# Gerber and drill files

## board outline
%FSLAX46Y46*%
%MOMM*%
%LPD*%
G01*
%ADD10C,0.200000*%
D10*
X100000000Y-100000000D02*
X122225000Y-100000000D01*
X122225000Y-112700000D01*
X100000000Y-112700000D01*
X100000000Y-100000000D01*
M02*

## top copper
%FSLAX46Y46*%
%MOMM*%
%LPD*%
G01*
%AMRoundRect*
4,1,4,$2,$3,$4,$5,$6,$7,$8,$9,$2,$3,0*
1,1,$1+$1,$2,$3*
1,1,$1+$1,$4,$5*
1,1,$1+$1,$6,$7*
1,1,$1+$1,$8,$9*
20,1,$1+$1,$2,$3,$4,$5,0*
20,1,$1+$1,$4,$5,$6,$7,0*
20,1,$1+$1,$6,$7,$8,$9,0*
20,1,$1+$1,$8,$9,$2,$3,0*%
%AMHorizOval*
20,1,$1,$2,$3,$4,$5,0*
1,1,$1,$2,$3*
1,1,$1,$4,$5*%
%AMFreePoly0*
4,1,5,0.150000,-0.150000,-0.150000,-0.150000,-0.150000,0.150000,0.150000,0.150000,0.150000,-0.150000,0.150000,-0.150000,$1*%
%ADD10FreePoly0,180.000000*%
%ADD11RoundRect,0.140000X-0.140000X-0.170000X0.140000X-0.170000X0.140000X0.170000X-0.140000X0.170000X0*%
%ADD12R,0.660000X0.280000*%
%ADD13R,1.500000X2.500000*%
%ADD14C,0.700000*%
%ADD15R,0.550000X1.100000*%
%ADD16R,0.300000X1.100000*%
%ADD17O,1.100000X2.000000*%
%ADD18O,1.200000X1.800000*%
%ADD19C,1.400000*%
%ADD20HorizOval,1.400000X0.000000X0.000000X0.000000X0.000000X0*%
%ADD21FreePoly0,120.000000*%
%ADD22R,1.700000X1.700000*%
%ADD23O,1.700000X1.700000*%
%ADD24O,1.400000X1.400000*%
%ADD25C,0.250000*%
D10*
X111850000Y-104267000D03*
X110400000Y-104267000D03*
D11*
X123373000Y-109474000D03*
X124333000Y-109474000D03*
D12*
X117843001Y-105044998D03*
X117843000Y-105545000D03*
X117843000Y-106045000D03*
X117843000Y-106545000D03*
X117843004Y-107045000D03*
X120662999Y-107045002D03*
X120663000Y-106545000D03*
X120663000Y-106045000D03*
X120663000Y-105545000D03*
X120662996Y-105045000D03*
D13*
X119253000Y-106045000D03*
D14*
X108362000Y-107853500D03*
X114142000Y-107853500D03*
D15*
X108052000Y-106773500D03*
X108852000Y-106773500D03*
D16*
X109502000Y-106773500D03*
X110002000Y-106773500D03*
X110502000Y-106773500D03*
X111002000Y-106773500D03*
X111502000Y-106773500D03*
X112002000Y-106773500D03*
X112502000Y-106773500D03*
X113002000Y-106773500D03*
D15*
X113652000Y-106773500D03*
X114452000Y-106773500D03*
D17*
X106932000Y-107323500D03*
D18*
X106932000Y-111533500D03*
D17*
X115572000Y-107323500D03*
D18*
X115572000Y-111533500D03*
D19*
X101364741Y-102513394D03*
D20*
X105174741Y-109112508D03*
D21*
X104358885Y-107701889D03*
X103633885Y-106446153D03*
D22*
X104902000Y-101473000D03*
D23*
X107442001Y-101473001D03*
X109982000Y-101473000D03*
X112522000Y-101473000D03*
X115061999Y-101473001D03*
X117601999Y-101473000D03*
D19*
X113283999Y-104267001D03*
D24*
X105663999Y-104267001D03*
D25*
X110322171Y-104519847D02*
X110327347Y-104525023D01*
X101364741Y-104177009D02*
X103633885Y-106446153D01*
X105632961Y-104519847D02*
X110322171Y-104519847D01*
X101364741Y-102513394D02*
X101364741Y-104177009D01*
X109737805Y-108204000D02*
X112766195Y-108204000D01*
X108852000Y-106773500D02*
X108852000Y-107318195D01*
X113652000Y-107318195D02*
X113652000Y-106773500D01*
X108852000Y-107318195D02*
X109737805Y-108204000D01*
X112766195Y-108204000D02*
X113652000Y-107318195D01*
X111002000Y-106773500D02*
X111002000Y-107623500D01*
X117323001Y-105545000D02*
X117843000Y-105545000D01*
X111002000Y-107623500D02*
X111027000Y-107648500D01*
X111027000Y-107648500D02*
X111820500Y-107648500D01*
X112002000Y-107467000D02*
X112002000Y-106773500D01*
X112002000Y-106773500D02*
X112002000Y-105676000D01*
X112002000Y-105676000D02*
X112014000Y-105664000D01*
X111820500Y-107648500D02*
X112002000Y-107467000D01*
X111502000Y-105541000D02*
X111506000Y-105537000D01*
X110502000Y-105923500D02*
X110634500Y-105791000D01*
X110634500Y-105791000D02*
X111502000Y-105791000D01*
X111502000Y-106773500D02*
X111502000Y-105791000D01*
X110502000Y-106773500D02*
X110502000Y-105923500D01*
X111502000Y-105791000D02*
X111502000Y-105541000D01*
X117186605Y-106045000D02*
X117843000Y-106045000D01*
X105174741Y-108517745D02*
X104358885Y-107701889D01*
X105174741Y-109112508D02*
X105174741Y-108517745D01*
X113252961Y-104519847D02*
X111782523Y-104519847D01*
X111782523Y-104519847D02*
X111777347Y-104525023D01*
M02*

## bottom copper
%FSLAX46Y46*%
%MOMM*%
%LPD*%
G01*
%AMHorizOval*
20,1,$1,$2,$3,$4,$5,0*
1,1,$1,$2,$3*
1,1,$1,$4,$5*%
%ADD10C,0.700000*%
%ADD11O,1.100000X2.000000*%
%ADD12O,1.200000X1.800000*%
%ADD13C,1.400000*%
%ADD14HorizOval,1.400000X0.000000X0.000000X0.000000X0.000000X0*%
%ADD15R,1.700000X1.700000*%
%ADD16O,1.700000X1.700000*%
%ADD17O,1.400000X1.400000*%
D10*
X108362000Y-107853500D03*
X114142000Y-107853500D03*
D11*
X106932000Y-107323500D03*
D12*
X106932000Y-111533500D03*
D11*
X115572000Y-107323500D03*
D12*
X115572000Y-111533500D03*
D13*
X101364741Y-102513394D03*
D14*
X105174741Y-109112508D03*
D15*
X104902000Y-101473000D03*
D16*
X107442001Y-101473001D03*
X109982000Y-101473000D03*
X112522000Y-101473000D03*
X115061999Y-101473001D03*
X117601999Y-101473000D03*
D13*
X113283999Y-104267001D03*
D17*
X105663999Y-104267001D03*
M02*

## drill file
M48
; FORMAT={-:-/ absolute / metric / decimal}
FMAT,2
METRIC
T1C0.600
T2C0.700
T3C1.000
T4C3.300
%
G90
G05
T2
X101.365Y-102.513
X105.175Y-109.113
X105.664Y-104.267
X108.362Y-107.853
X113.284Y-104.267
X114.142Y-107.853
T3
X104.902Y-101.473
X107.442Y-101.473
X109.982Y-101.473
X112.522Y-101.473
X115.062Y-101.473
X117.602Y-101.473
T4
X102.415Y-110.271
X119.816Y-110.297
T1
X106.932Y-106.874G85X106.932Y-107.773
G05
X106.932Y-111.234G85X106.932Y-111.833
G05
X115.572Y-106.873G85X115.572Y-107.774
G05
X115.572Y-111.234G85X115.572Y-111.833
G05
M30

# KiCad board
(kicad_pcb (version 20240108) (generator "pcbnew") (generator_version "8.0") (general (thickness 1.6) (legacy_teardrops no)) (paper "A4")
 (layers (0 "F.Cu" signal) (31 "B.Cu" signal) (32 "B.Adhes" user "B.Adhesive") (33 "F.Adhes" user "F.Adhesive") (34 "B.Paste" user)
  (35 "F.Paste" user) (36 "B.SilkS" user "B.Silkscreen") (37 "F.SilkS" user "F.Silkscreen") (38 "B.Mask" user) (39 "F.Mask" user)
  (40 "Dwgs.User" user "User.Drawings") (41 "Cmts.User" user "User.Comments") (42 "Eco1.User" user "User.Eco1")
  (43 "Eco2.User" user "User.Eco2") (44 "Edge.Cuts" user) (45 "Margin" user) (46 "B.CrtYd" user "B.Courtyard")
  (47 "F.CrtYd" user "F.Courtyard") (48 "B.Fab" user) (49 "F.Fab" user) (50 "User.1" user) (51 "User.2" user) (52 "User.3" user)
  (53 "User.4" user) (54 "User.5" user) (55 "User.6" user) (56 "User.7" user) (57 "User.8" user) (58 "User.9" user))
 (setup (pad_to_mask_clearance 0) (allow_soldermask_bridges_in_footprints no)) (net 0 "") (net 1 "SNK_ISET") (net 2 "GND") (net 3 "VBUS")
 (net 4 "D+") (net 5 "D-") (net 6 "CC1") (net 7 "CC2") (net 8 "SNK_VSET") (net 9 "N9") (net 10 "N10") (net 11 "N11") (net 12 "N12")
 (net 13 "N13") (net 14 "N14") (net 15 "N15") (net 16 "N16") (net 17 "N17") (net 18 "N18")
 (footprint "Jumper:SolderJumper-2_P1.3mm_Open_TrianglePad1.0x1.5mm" (layer "F.Cu") (at 111.125 104.267 180)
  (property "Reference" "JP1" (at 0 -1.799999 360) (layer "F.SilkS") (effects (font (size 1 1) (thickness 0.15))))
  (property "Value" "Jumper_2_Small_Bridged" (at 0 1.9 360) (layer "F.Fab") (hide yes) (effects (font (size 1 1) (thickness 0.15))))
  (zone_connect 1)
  (pad "1" smd custom (at -0.725 0 180) (size 0.3 0.3) (layers "F.Cu" "F.Mask") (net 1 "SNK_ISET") (zone_connect 2)
   (thermal_bridge_angle 45) (options (clearance outline) (anchor rect)) (primitives))
  (pad "2" smd custom (at 0.725 0 180) (size 0.3 0.3) (layers "F.Cu" "F.Mask") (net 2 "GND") (zone_connect 2) (thermal_bridge_angle 45)
   (options (clearance outline) (anchor rect)) (primitives)))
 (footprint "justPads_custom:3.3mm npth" (layer "F.Cu") (at 102.415229 110.27145)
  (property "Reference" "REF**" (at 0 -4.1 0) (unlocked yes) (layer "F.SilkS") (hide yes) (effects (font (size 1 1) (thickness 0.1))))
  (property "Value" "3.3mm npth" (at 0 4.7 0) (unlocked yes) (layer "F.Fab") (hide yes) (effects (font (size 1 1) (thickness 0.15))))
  (pad "" np_thru_hole circle (at 0 0) (size 3.3 3.3) (drill 3.3) (layers "F&B.Cu" "*.Mask")))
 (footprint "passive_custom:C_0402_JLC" (layer "F.Cu") (at 123.8356 109.478)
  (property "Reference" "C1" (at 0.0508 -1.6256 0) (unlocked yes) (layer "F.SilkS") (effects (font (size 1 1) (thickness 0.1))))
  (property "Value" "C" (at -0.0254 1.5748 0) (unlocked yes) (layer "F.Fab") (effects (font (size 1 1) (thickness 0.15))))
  (pad "1" smd roundrect (at -0.4626 -0.004) (size 0.56 0.62) (layers "F.Cu" "F.Paste" "F.Mask") (roundrect_rratio 0.25) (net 2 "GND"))
  (pad "2" smd roundrect (at 0.4974 -0.004) (size 0.56 0.62) (layers "F.Cu" "F.Paste" "F.Mask") (roundrect_rratio 0.25) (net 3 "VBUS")))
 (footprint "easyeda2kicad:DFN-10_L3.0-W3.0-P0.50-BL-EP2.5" (layer "F.Cu") (at 119.253 106.045 -90)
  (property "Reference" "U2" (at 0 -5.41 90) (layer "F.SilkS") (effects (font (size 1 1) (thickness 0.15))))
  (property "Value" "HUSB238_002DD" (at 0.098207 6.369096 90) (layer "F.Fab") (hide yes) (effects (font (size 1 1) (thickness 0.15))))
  (pad "1" smd rect (at -1.000002 1.409999 270) (size 0.28 0.66) (layers "F.Cu" "F.Paste" "F.Mask") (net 3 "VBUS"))
  (pad "2" smd rect (at -0.5 1.41 270) (size 0.28 0.66) (layers "F.Cu" "F.Paste" "F.Mask") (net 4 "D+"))
  (pad "3" smd rect (at 0 1.41 270) (size 0.28 0.66) (layers "F.Cu" "F.Paste" "F.Mask") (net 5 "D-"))
  (pad "4" smd rect (at 0.5 1.41 270) (size 0.28 0.66) (layers "F.Cu" "F.Paste" "F.Mask") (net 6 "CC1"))
  (pad "5" smd rect (at 1 1.409996 270) (size 0.28 0.66) (layers "F.Cu" "F.Paste" "F.Mask") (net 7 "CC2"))
  (pad "6" smd rect (at 1.000002 -1.409999 270) (size 0.28 0.66) (layers "F.Cu" "F.Paste" "F.Mask") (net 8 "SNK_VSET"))
  (pad "7" smd rect (at 0.5 -1.41 270) (size 0.28 0.66) (layers "F.Cu" "F.Paste" "F.Mask") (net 1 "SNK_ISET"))
  (pad "8" smd rect (at 0 -1.41 270) (size 0.28 0.66) (layers "F.Cu" "F.Paste" "F.Mask") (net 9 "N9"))
  (pad "9" smd rect (at -0.5 -1.41 270) (size 0.28 0.66) (layers "F.Cu" "F.Paste" "F.Mask") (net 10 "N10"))
  (pad "10" smd rect (at -1 -1.409996 270) (size 0.28 0.66) (layers "F.Cu" "F.Paste" "F.Mask") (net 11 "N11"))
  (pad "11" smd rect (at 0 0 270) (size 2.5 1.5) (layers "F.Cu" "F.Paste" "F.Mask") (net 2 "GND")))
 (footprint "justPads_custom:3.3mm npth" (layer "F.Cu") (at 119.816242 110.29744)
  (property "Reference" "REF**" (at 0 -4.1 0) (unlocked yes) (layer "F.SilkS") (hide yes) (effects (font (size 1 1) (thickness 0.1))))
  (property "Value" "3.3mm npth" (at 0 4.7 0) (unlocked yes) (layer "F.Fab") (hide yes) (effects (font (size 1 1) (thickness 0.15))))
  (pad "" np_thru_hole circle (at 0 0) (size 3.3 3.3) (drill 3.3) (layers "F&B.Cu" "*.Mask")))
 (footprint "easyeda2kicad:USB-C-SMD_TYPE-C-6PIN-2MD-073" (layer "F.Cu") (at 111.252 109.1535)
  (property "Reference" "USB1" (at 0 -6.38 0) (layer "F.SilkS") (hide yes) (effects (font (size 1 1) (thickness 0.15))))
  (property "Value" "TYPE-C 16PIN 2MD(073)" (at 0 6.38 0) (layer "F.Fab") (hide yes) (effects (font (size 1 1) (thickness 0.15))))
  (pad "" thru_hole circle (at -2.89 -1.3) (size 0.7 0.7) (drill 0.7) (layers "*.Cu" "*.Mask") (remove_unused_layers no))
  (pad "" thru_hole circle (at 2.89 -1.3) (size 0.7 0.7) (drill 0.7) (layers "*.Cu" "*.Mask") (remove_unused_layers no))
  (pad "1" smd rect (at -3.2 -2.38) (size 0.55 1.1) (layers "F.Cu" "F.Paste" "F.Mask") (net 2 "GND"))
  (pad "2" smd rect (at -2.4 -2.38) (size 0.55 1.1) (layers "F.Cu" "F.Paste" "F.Mask") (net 3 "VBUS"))
  (pad "3" smd rect (at -1.75 -2.38) (size 0.3 1.1) (layers "F.Cu" "F.Paste" "F.Mask") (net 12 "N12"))
  (pad "4" smd rect (at -1.25 -2.38) (size 0.3 1.1) (layers "F.Cu" "F.Paste" "F.Mask") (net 6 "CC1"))
  (pad "5" smd rect (at -0.75 -2.38) (size 0.3 1.1) (layers "F.Cu" "F.Paste" "F.Mask") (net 5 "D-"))
  (pad "6" smd rect (at -0.25 -2.38) (size 0.3 1.1) (layers "F.Cu" "F.Paste" "F.Mask") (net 4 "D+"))
  (pad "7" smd rect (at 0.25 -2.38) (size 0.3 1.1) (layers "F.Cu" "F.Paste" "F.Mask") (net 5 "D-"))
  (pad "8" smd rect (at 0.75 -2.38) (size 0.3 1.1) (layers "F.Cu" "F.Paste" "F.Mask") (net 4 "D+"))
  (pad "9" smd rect (at 1.25 -2.38) (size 0.3 1.1) (layers "F.Cu" "F.Paste" "F.Mask") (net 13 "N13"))
  (pad "10" smd rect (at 1.75 -2.38) (size 0.3 1.1) (layers "F.Cu" "F.Paste" "F.Mask") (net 7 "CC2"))
  (pad "11" smd rect (at 2.4 -2.38) (size 0.55 1.1) (layers "F.Cu" "F.Paste" "F.Mask") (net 3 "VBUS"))
  (pad "12" smd rect (at 3.2 -2.38) (size 0.55 1.1) (layers "F.Cu" "F.Paste" "F.Mask") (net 2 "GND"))
  (pad "13" thru_hole oval (at -4.32 -1.83) (size 1.1 2) (drill oval 0.599999 1.499997) (layers "*.Cu" "*.Mask") (remove_unused_layers no)
   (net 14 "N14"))
  (pad "13" thru_hole oval (at -4.32 2.38) (size 1.2 1.8) (drill oval 0.599999 1.199998) (layers "*.Cu" "*.Mask") (remove_unused_layers no)
   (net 14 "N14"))
  (pad "14" thru_hole oval (at 4.32 -1.83) (size 1.1 2) (drill oval 0.599999 1.500022) (layers "*.Cu" "*.Mask") (remove_unused_layers no)
   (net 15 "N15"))
  (pad "14" thru_hole oval (at 4.32 2.38) (size 1.2 1.8) (drill oval 0.599999 1.199998) (layers "*.Cu" "*.Mask") (remove_unused_layers no)
   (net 15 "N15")))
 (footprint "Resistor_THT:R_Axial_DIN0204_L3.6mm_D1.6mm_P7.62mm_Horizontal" (layer "F.Cu") (at 101.364741 102.513394 -60)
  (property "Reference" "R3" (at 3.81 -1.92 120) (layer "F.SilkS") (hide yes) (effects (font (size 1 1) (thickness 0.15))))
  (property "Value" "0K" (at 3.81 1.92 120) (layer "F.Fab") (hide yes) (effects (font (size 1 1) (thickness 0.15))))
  (pad "1" thru_hole circle (at 0 0 300) (size 1.4 1.4) (drill 0.7) (layers "*.Cu" "*.Mask") (remove_unused_layers no) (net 2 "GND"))
  (pad "2" thru_hole oval (at 7.62 0 300) (size 1.4 1.4) (drill 0.7) (layers "*.Cu" "*.Mask") (remove_unused_layers no) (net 8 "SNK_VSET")))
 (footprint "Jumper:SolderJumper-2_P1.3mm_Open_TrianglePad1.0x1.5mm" (layer "F.Cu") (at 103.996385 107.074021 120)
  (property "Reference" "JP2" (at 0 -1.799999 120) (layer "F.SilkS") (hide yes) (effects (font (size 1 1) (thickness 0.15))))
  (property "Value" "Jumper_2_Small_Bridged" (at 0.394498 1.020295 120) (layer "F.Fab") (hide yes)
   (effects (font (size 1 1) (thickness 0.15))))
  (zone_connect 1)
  (pad "1" smd custom (at -0.725 0 120) (size 0.3 0.3) (layers "F.Cu" "F.Mask") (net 8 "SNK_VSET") (zone_connect 2)
   (thermal_bridge_angle 45) (options (clearance outline) (anchor rect)) (primitives))
  (pad "2" smd custom (at 0.725 0 120) (size 0.3 0.3) (layers "F.Cu" "F.Mask") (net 2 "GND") (zone_connect 2) (thermal_bridge_angle 45)
   (options (clearance outline) (anchor rect)) (primitives)))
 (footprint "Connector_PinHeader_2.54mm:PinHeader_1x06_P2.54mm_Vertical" (layer "F.Cu") (at 104.902 101.473 90)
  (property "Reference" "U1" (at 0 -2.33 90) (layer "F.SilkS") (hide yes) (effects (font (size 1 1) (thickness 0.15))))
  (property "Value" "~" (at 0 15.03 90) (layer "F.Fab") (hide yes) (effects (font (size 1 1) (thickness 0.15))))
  (pad "1" thru_hole rect (at 0 0 90) (size 1.7 1.7) (drill 1) (layers "*.Cu" "*.Mask") (remove_unused_layers no) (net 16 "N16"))
  (pad "2" thru_hole oval (at -0.000001 2.540001 90) (size 1.7 1.7) (drill 1) (layers "*.Cu" "*.Mask") (remove_unused_layers no)
   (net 2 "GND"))
  (pad "3" thru_hole oval (at 0 5.08 90) (size 1.7 1.7) (drill 1) (layers "*.Cu" "*.Mask") (remove_unused_layers no) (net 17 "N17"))
  (pad "4" thru_hole oval (at 0 7.62 90) (size 1.7 1.7) (drill 1) (layers "*.Cu" "*.Mask") (remove_unused_layers no) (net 5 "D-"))
  (pad "5" thru_hole oval (at -0.000001 10.159999 90) (size 1.7 1.7) (drill 1) (layers "*.Cu" "*.Mask") (remove_unused_layers no)
   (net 4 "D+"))
  (pad "6" thru_hole oval (at 0 12.699999 90) (size 1.7 1.7) (drill 1) (layers "*.Cu" "*.Mask") (remove_unused_layers no) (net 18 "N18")))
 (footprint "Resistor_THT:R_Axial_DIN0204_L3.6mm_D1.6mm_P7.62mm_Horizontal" (layer "F.Cu") (at 113.283999 104.267001 180)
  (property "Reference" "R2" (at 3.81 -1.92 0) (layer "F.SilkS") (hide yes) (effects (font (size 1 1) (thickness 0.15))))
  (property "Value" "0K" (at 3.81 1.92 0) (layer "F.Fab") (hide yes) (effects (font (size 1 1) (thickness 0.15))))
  (pad "1" thru_hole circle (at 0 0 180) (size 1.4 1.4) (drill 0.7) (layers "*.Cu" "*.Mask") (remove_unused_layers no) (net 1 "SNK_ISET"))
  (pad "2" thru_hole oval (at 7.62 0 180) (size 1.4 1.4) (drill 0.7) (layers "*.Cu" "*.Mask") (remove_unused_layers no) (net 2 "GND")))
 (gr_rect (start 100 100) (end 122.225 112.7) (stroke (width 0.2) (type default)) (fill none) (layer "Edge.Cuts"))
 (segment (start 110.322171 104.519847) (end 110.327347 104.525023) (width 0.25) (layer "F.Cu") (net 2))
 (segment (start 101.364741 104.177009) (end 103.633885 106.446153) (width 0.25) (layer "F.Cu") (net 2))
 (segment (start 105.632961 104.519847) (end 110.322171 104.519847) (width 0.25) (layer "F.Cu") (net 2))
 (segment (start 101.364741 102.513394) (end 101.364741 104.177009) (width 0.25) (layer "F.Cu") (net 2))
 (segment (start 109.737805 108.204) (end 112.766195 108.204) (width 0.25) (layer "F.Cu") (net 3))
 (segment (start 108.852 106.7735) (end 108.852 107.318195) (width 0.25) (layer "F.Cu") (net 3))
 (segment (start 113.652 107.318195) (end 113.652 106.7735) (width 0.25) (layer "F.Cu") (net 3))
 (segment (start 108.852 107.318195) (end 109.737805 108.204) (width 0.25) (layer "F.Cu") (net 3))
 (segment (start 112.766195 108.204) (end 113.652 107.318195) (width 0.25) (layer "F.Cu") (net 3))
 (segment (start 111.002 106.7735) (end 111.002 107.6235) (width 0.25) (layer "F.Cu") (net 4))
 (segment (start 117.323001 105.545) (end 117.843 105.545) (width 0.25) (layer "F.Cu") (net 4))
 (segment (start 111.002 107.6235) (end 111.027 107.6485) (width 0.25) (layer "F.Cu") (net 4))
 (segment (start 111.027 107.6485) (end 111.8205 107.6485) (width 0.25) (layer "F.Cu") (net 4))
 (segment (start 112.002 107.467) (end 112.002 106.7735) (width 0.25) (layer "F.Cu") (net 4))
 (segment (start 112.002 106.7735) (end 112.002 105.676) (width 0.25) (layer "F.Cu") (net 4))
 (segment (start 112.002 105.676) (end 112.014 105.664) (width 0.25) (layer "F.Cu") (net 4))
 (segment (start 111.8205 107.6485) (end 112.002 107.467) (width 0.25) (layer "F.Cu") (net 4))
 (segment (start 111.502 105.541) (end 111.506 105.537) (width 0.25) (layer "F.Cu") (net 5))
 (segment (start 110.502 105.9235) (end 110.6345 105.791) (width 0.25) (layer "F.Cu") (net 5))
 (segment (start 110.6345 105.791) (end 111.502 105.791) (width 0.25) (layer "F.Cu") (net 5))
 (segment (start 111.502 106.7735) (end 111.502 105.791) (width 0.25) (layer "F.Cu") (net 5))
 (segment (start 110.502 106.7735) (end 110.502 105.9235) (width 0.25) (layer "F.Cu") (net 5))
 (segment (start 111.502 105.791) (end 111.502 105.541) (width 0.25) (layer "F.Cu") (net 5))
 (segment (start 117.186605 106.045) (end 117.843 106.045) (width 0.25) (layer "F.Cu") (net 5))
 (segment (start 105.174741 108.517745) (end 104.358885 107.701889) (width 0.25) (layer "F.Cu") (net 8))
 (segment (start 105.174741 109.112508) (end 105.174741 108.517745) (width 0.25) (layer "F.Cu") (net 8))
 (segment (start 113.252961 104.519847) (end 111.782523 104.519847) (width 0.25) (layer "F.Cu") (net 1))
 (segment (start 111.782523 104.519847) (end 111.777347 104.525023) (width 0.25) (layer "F.Cu") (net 1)))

